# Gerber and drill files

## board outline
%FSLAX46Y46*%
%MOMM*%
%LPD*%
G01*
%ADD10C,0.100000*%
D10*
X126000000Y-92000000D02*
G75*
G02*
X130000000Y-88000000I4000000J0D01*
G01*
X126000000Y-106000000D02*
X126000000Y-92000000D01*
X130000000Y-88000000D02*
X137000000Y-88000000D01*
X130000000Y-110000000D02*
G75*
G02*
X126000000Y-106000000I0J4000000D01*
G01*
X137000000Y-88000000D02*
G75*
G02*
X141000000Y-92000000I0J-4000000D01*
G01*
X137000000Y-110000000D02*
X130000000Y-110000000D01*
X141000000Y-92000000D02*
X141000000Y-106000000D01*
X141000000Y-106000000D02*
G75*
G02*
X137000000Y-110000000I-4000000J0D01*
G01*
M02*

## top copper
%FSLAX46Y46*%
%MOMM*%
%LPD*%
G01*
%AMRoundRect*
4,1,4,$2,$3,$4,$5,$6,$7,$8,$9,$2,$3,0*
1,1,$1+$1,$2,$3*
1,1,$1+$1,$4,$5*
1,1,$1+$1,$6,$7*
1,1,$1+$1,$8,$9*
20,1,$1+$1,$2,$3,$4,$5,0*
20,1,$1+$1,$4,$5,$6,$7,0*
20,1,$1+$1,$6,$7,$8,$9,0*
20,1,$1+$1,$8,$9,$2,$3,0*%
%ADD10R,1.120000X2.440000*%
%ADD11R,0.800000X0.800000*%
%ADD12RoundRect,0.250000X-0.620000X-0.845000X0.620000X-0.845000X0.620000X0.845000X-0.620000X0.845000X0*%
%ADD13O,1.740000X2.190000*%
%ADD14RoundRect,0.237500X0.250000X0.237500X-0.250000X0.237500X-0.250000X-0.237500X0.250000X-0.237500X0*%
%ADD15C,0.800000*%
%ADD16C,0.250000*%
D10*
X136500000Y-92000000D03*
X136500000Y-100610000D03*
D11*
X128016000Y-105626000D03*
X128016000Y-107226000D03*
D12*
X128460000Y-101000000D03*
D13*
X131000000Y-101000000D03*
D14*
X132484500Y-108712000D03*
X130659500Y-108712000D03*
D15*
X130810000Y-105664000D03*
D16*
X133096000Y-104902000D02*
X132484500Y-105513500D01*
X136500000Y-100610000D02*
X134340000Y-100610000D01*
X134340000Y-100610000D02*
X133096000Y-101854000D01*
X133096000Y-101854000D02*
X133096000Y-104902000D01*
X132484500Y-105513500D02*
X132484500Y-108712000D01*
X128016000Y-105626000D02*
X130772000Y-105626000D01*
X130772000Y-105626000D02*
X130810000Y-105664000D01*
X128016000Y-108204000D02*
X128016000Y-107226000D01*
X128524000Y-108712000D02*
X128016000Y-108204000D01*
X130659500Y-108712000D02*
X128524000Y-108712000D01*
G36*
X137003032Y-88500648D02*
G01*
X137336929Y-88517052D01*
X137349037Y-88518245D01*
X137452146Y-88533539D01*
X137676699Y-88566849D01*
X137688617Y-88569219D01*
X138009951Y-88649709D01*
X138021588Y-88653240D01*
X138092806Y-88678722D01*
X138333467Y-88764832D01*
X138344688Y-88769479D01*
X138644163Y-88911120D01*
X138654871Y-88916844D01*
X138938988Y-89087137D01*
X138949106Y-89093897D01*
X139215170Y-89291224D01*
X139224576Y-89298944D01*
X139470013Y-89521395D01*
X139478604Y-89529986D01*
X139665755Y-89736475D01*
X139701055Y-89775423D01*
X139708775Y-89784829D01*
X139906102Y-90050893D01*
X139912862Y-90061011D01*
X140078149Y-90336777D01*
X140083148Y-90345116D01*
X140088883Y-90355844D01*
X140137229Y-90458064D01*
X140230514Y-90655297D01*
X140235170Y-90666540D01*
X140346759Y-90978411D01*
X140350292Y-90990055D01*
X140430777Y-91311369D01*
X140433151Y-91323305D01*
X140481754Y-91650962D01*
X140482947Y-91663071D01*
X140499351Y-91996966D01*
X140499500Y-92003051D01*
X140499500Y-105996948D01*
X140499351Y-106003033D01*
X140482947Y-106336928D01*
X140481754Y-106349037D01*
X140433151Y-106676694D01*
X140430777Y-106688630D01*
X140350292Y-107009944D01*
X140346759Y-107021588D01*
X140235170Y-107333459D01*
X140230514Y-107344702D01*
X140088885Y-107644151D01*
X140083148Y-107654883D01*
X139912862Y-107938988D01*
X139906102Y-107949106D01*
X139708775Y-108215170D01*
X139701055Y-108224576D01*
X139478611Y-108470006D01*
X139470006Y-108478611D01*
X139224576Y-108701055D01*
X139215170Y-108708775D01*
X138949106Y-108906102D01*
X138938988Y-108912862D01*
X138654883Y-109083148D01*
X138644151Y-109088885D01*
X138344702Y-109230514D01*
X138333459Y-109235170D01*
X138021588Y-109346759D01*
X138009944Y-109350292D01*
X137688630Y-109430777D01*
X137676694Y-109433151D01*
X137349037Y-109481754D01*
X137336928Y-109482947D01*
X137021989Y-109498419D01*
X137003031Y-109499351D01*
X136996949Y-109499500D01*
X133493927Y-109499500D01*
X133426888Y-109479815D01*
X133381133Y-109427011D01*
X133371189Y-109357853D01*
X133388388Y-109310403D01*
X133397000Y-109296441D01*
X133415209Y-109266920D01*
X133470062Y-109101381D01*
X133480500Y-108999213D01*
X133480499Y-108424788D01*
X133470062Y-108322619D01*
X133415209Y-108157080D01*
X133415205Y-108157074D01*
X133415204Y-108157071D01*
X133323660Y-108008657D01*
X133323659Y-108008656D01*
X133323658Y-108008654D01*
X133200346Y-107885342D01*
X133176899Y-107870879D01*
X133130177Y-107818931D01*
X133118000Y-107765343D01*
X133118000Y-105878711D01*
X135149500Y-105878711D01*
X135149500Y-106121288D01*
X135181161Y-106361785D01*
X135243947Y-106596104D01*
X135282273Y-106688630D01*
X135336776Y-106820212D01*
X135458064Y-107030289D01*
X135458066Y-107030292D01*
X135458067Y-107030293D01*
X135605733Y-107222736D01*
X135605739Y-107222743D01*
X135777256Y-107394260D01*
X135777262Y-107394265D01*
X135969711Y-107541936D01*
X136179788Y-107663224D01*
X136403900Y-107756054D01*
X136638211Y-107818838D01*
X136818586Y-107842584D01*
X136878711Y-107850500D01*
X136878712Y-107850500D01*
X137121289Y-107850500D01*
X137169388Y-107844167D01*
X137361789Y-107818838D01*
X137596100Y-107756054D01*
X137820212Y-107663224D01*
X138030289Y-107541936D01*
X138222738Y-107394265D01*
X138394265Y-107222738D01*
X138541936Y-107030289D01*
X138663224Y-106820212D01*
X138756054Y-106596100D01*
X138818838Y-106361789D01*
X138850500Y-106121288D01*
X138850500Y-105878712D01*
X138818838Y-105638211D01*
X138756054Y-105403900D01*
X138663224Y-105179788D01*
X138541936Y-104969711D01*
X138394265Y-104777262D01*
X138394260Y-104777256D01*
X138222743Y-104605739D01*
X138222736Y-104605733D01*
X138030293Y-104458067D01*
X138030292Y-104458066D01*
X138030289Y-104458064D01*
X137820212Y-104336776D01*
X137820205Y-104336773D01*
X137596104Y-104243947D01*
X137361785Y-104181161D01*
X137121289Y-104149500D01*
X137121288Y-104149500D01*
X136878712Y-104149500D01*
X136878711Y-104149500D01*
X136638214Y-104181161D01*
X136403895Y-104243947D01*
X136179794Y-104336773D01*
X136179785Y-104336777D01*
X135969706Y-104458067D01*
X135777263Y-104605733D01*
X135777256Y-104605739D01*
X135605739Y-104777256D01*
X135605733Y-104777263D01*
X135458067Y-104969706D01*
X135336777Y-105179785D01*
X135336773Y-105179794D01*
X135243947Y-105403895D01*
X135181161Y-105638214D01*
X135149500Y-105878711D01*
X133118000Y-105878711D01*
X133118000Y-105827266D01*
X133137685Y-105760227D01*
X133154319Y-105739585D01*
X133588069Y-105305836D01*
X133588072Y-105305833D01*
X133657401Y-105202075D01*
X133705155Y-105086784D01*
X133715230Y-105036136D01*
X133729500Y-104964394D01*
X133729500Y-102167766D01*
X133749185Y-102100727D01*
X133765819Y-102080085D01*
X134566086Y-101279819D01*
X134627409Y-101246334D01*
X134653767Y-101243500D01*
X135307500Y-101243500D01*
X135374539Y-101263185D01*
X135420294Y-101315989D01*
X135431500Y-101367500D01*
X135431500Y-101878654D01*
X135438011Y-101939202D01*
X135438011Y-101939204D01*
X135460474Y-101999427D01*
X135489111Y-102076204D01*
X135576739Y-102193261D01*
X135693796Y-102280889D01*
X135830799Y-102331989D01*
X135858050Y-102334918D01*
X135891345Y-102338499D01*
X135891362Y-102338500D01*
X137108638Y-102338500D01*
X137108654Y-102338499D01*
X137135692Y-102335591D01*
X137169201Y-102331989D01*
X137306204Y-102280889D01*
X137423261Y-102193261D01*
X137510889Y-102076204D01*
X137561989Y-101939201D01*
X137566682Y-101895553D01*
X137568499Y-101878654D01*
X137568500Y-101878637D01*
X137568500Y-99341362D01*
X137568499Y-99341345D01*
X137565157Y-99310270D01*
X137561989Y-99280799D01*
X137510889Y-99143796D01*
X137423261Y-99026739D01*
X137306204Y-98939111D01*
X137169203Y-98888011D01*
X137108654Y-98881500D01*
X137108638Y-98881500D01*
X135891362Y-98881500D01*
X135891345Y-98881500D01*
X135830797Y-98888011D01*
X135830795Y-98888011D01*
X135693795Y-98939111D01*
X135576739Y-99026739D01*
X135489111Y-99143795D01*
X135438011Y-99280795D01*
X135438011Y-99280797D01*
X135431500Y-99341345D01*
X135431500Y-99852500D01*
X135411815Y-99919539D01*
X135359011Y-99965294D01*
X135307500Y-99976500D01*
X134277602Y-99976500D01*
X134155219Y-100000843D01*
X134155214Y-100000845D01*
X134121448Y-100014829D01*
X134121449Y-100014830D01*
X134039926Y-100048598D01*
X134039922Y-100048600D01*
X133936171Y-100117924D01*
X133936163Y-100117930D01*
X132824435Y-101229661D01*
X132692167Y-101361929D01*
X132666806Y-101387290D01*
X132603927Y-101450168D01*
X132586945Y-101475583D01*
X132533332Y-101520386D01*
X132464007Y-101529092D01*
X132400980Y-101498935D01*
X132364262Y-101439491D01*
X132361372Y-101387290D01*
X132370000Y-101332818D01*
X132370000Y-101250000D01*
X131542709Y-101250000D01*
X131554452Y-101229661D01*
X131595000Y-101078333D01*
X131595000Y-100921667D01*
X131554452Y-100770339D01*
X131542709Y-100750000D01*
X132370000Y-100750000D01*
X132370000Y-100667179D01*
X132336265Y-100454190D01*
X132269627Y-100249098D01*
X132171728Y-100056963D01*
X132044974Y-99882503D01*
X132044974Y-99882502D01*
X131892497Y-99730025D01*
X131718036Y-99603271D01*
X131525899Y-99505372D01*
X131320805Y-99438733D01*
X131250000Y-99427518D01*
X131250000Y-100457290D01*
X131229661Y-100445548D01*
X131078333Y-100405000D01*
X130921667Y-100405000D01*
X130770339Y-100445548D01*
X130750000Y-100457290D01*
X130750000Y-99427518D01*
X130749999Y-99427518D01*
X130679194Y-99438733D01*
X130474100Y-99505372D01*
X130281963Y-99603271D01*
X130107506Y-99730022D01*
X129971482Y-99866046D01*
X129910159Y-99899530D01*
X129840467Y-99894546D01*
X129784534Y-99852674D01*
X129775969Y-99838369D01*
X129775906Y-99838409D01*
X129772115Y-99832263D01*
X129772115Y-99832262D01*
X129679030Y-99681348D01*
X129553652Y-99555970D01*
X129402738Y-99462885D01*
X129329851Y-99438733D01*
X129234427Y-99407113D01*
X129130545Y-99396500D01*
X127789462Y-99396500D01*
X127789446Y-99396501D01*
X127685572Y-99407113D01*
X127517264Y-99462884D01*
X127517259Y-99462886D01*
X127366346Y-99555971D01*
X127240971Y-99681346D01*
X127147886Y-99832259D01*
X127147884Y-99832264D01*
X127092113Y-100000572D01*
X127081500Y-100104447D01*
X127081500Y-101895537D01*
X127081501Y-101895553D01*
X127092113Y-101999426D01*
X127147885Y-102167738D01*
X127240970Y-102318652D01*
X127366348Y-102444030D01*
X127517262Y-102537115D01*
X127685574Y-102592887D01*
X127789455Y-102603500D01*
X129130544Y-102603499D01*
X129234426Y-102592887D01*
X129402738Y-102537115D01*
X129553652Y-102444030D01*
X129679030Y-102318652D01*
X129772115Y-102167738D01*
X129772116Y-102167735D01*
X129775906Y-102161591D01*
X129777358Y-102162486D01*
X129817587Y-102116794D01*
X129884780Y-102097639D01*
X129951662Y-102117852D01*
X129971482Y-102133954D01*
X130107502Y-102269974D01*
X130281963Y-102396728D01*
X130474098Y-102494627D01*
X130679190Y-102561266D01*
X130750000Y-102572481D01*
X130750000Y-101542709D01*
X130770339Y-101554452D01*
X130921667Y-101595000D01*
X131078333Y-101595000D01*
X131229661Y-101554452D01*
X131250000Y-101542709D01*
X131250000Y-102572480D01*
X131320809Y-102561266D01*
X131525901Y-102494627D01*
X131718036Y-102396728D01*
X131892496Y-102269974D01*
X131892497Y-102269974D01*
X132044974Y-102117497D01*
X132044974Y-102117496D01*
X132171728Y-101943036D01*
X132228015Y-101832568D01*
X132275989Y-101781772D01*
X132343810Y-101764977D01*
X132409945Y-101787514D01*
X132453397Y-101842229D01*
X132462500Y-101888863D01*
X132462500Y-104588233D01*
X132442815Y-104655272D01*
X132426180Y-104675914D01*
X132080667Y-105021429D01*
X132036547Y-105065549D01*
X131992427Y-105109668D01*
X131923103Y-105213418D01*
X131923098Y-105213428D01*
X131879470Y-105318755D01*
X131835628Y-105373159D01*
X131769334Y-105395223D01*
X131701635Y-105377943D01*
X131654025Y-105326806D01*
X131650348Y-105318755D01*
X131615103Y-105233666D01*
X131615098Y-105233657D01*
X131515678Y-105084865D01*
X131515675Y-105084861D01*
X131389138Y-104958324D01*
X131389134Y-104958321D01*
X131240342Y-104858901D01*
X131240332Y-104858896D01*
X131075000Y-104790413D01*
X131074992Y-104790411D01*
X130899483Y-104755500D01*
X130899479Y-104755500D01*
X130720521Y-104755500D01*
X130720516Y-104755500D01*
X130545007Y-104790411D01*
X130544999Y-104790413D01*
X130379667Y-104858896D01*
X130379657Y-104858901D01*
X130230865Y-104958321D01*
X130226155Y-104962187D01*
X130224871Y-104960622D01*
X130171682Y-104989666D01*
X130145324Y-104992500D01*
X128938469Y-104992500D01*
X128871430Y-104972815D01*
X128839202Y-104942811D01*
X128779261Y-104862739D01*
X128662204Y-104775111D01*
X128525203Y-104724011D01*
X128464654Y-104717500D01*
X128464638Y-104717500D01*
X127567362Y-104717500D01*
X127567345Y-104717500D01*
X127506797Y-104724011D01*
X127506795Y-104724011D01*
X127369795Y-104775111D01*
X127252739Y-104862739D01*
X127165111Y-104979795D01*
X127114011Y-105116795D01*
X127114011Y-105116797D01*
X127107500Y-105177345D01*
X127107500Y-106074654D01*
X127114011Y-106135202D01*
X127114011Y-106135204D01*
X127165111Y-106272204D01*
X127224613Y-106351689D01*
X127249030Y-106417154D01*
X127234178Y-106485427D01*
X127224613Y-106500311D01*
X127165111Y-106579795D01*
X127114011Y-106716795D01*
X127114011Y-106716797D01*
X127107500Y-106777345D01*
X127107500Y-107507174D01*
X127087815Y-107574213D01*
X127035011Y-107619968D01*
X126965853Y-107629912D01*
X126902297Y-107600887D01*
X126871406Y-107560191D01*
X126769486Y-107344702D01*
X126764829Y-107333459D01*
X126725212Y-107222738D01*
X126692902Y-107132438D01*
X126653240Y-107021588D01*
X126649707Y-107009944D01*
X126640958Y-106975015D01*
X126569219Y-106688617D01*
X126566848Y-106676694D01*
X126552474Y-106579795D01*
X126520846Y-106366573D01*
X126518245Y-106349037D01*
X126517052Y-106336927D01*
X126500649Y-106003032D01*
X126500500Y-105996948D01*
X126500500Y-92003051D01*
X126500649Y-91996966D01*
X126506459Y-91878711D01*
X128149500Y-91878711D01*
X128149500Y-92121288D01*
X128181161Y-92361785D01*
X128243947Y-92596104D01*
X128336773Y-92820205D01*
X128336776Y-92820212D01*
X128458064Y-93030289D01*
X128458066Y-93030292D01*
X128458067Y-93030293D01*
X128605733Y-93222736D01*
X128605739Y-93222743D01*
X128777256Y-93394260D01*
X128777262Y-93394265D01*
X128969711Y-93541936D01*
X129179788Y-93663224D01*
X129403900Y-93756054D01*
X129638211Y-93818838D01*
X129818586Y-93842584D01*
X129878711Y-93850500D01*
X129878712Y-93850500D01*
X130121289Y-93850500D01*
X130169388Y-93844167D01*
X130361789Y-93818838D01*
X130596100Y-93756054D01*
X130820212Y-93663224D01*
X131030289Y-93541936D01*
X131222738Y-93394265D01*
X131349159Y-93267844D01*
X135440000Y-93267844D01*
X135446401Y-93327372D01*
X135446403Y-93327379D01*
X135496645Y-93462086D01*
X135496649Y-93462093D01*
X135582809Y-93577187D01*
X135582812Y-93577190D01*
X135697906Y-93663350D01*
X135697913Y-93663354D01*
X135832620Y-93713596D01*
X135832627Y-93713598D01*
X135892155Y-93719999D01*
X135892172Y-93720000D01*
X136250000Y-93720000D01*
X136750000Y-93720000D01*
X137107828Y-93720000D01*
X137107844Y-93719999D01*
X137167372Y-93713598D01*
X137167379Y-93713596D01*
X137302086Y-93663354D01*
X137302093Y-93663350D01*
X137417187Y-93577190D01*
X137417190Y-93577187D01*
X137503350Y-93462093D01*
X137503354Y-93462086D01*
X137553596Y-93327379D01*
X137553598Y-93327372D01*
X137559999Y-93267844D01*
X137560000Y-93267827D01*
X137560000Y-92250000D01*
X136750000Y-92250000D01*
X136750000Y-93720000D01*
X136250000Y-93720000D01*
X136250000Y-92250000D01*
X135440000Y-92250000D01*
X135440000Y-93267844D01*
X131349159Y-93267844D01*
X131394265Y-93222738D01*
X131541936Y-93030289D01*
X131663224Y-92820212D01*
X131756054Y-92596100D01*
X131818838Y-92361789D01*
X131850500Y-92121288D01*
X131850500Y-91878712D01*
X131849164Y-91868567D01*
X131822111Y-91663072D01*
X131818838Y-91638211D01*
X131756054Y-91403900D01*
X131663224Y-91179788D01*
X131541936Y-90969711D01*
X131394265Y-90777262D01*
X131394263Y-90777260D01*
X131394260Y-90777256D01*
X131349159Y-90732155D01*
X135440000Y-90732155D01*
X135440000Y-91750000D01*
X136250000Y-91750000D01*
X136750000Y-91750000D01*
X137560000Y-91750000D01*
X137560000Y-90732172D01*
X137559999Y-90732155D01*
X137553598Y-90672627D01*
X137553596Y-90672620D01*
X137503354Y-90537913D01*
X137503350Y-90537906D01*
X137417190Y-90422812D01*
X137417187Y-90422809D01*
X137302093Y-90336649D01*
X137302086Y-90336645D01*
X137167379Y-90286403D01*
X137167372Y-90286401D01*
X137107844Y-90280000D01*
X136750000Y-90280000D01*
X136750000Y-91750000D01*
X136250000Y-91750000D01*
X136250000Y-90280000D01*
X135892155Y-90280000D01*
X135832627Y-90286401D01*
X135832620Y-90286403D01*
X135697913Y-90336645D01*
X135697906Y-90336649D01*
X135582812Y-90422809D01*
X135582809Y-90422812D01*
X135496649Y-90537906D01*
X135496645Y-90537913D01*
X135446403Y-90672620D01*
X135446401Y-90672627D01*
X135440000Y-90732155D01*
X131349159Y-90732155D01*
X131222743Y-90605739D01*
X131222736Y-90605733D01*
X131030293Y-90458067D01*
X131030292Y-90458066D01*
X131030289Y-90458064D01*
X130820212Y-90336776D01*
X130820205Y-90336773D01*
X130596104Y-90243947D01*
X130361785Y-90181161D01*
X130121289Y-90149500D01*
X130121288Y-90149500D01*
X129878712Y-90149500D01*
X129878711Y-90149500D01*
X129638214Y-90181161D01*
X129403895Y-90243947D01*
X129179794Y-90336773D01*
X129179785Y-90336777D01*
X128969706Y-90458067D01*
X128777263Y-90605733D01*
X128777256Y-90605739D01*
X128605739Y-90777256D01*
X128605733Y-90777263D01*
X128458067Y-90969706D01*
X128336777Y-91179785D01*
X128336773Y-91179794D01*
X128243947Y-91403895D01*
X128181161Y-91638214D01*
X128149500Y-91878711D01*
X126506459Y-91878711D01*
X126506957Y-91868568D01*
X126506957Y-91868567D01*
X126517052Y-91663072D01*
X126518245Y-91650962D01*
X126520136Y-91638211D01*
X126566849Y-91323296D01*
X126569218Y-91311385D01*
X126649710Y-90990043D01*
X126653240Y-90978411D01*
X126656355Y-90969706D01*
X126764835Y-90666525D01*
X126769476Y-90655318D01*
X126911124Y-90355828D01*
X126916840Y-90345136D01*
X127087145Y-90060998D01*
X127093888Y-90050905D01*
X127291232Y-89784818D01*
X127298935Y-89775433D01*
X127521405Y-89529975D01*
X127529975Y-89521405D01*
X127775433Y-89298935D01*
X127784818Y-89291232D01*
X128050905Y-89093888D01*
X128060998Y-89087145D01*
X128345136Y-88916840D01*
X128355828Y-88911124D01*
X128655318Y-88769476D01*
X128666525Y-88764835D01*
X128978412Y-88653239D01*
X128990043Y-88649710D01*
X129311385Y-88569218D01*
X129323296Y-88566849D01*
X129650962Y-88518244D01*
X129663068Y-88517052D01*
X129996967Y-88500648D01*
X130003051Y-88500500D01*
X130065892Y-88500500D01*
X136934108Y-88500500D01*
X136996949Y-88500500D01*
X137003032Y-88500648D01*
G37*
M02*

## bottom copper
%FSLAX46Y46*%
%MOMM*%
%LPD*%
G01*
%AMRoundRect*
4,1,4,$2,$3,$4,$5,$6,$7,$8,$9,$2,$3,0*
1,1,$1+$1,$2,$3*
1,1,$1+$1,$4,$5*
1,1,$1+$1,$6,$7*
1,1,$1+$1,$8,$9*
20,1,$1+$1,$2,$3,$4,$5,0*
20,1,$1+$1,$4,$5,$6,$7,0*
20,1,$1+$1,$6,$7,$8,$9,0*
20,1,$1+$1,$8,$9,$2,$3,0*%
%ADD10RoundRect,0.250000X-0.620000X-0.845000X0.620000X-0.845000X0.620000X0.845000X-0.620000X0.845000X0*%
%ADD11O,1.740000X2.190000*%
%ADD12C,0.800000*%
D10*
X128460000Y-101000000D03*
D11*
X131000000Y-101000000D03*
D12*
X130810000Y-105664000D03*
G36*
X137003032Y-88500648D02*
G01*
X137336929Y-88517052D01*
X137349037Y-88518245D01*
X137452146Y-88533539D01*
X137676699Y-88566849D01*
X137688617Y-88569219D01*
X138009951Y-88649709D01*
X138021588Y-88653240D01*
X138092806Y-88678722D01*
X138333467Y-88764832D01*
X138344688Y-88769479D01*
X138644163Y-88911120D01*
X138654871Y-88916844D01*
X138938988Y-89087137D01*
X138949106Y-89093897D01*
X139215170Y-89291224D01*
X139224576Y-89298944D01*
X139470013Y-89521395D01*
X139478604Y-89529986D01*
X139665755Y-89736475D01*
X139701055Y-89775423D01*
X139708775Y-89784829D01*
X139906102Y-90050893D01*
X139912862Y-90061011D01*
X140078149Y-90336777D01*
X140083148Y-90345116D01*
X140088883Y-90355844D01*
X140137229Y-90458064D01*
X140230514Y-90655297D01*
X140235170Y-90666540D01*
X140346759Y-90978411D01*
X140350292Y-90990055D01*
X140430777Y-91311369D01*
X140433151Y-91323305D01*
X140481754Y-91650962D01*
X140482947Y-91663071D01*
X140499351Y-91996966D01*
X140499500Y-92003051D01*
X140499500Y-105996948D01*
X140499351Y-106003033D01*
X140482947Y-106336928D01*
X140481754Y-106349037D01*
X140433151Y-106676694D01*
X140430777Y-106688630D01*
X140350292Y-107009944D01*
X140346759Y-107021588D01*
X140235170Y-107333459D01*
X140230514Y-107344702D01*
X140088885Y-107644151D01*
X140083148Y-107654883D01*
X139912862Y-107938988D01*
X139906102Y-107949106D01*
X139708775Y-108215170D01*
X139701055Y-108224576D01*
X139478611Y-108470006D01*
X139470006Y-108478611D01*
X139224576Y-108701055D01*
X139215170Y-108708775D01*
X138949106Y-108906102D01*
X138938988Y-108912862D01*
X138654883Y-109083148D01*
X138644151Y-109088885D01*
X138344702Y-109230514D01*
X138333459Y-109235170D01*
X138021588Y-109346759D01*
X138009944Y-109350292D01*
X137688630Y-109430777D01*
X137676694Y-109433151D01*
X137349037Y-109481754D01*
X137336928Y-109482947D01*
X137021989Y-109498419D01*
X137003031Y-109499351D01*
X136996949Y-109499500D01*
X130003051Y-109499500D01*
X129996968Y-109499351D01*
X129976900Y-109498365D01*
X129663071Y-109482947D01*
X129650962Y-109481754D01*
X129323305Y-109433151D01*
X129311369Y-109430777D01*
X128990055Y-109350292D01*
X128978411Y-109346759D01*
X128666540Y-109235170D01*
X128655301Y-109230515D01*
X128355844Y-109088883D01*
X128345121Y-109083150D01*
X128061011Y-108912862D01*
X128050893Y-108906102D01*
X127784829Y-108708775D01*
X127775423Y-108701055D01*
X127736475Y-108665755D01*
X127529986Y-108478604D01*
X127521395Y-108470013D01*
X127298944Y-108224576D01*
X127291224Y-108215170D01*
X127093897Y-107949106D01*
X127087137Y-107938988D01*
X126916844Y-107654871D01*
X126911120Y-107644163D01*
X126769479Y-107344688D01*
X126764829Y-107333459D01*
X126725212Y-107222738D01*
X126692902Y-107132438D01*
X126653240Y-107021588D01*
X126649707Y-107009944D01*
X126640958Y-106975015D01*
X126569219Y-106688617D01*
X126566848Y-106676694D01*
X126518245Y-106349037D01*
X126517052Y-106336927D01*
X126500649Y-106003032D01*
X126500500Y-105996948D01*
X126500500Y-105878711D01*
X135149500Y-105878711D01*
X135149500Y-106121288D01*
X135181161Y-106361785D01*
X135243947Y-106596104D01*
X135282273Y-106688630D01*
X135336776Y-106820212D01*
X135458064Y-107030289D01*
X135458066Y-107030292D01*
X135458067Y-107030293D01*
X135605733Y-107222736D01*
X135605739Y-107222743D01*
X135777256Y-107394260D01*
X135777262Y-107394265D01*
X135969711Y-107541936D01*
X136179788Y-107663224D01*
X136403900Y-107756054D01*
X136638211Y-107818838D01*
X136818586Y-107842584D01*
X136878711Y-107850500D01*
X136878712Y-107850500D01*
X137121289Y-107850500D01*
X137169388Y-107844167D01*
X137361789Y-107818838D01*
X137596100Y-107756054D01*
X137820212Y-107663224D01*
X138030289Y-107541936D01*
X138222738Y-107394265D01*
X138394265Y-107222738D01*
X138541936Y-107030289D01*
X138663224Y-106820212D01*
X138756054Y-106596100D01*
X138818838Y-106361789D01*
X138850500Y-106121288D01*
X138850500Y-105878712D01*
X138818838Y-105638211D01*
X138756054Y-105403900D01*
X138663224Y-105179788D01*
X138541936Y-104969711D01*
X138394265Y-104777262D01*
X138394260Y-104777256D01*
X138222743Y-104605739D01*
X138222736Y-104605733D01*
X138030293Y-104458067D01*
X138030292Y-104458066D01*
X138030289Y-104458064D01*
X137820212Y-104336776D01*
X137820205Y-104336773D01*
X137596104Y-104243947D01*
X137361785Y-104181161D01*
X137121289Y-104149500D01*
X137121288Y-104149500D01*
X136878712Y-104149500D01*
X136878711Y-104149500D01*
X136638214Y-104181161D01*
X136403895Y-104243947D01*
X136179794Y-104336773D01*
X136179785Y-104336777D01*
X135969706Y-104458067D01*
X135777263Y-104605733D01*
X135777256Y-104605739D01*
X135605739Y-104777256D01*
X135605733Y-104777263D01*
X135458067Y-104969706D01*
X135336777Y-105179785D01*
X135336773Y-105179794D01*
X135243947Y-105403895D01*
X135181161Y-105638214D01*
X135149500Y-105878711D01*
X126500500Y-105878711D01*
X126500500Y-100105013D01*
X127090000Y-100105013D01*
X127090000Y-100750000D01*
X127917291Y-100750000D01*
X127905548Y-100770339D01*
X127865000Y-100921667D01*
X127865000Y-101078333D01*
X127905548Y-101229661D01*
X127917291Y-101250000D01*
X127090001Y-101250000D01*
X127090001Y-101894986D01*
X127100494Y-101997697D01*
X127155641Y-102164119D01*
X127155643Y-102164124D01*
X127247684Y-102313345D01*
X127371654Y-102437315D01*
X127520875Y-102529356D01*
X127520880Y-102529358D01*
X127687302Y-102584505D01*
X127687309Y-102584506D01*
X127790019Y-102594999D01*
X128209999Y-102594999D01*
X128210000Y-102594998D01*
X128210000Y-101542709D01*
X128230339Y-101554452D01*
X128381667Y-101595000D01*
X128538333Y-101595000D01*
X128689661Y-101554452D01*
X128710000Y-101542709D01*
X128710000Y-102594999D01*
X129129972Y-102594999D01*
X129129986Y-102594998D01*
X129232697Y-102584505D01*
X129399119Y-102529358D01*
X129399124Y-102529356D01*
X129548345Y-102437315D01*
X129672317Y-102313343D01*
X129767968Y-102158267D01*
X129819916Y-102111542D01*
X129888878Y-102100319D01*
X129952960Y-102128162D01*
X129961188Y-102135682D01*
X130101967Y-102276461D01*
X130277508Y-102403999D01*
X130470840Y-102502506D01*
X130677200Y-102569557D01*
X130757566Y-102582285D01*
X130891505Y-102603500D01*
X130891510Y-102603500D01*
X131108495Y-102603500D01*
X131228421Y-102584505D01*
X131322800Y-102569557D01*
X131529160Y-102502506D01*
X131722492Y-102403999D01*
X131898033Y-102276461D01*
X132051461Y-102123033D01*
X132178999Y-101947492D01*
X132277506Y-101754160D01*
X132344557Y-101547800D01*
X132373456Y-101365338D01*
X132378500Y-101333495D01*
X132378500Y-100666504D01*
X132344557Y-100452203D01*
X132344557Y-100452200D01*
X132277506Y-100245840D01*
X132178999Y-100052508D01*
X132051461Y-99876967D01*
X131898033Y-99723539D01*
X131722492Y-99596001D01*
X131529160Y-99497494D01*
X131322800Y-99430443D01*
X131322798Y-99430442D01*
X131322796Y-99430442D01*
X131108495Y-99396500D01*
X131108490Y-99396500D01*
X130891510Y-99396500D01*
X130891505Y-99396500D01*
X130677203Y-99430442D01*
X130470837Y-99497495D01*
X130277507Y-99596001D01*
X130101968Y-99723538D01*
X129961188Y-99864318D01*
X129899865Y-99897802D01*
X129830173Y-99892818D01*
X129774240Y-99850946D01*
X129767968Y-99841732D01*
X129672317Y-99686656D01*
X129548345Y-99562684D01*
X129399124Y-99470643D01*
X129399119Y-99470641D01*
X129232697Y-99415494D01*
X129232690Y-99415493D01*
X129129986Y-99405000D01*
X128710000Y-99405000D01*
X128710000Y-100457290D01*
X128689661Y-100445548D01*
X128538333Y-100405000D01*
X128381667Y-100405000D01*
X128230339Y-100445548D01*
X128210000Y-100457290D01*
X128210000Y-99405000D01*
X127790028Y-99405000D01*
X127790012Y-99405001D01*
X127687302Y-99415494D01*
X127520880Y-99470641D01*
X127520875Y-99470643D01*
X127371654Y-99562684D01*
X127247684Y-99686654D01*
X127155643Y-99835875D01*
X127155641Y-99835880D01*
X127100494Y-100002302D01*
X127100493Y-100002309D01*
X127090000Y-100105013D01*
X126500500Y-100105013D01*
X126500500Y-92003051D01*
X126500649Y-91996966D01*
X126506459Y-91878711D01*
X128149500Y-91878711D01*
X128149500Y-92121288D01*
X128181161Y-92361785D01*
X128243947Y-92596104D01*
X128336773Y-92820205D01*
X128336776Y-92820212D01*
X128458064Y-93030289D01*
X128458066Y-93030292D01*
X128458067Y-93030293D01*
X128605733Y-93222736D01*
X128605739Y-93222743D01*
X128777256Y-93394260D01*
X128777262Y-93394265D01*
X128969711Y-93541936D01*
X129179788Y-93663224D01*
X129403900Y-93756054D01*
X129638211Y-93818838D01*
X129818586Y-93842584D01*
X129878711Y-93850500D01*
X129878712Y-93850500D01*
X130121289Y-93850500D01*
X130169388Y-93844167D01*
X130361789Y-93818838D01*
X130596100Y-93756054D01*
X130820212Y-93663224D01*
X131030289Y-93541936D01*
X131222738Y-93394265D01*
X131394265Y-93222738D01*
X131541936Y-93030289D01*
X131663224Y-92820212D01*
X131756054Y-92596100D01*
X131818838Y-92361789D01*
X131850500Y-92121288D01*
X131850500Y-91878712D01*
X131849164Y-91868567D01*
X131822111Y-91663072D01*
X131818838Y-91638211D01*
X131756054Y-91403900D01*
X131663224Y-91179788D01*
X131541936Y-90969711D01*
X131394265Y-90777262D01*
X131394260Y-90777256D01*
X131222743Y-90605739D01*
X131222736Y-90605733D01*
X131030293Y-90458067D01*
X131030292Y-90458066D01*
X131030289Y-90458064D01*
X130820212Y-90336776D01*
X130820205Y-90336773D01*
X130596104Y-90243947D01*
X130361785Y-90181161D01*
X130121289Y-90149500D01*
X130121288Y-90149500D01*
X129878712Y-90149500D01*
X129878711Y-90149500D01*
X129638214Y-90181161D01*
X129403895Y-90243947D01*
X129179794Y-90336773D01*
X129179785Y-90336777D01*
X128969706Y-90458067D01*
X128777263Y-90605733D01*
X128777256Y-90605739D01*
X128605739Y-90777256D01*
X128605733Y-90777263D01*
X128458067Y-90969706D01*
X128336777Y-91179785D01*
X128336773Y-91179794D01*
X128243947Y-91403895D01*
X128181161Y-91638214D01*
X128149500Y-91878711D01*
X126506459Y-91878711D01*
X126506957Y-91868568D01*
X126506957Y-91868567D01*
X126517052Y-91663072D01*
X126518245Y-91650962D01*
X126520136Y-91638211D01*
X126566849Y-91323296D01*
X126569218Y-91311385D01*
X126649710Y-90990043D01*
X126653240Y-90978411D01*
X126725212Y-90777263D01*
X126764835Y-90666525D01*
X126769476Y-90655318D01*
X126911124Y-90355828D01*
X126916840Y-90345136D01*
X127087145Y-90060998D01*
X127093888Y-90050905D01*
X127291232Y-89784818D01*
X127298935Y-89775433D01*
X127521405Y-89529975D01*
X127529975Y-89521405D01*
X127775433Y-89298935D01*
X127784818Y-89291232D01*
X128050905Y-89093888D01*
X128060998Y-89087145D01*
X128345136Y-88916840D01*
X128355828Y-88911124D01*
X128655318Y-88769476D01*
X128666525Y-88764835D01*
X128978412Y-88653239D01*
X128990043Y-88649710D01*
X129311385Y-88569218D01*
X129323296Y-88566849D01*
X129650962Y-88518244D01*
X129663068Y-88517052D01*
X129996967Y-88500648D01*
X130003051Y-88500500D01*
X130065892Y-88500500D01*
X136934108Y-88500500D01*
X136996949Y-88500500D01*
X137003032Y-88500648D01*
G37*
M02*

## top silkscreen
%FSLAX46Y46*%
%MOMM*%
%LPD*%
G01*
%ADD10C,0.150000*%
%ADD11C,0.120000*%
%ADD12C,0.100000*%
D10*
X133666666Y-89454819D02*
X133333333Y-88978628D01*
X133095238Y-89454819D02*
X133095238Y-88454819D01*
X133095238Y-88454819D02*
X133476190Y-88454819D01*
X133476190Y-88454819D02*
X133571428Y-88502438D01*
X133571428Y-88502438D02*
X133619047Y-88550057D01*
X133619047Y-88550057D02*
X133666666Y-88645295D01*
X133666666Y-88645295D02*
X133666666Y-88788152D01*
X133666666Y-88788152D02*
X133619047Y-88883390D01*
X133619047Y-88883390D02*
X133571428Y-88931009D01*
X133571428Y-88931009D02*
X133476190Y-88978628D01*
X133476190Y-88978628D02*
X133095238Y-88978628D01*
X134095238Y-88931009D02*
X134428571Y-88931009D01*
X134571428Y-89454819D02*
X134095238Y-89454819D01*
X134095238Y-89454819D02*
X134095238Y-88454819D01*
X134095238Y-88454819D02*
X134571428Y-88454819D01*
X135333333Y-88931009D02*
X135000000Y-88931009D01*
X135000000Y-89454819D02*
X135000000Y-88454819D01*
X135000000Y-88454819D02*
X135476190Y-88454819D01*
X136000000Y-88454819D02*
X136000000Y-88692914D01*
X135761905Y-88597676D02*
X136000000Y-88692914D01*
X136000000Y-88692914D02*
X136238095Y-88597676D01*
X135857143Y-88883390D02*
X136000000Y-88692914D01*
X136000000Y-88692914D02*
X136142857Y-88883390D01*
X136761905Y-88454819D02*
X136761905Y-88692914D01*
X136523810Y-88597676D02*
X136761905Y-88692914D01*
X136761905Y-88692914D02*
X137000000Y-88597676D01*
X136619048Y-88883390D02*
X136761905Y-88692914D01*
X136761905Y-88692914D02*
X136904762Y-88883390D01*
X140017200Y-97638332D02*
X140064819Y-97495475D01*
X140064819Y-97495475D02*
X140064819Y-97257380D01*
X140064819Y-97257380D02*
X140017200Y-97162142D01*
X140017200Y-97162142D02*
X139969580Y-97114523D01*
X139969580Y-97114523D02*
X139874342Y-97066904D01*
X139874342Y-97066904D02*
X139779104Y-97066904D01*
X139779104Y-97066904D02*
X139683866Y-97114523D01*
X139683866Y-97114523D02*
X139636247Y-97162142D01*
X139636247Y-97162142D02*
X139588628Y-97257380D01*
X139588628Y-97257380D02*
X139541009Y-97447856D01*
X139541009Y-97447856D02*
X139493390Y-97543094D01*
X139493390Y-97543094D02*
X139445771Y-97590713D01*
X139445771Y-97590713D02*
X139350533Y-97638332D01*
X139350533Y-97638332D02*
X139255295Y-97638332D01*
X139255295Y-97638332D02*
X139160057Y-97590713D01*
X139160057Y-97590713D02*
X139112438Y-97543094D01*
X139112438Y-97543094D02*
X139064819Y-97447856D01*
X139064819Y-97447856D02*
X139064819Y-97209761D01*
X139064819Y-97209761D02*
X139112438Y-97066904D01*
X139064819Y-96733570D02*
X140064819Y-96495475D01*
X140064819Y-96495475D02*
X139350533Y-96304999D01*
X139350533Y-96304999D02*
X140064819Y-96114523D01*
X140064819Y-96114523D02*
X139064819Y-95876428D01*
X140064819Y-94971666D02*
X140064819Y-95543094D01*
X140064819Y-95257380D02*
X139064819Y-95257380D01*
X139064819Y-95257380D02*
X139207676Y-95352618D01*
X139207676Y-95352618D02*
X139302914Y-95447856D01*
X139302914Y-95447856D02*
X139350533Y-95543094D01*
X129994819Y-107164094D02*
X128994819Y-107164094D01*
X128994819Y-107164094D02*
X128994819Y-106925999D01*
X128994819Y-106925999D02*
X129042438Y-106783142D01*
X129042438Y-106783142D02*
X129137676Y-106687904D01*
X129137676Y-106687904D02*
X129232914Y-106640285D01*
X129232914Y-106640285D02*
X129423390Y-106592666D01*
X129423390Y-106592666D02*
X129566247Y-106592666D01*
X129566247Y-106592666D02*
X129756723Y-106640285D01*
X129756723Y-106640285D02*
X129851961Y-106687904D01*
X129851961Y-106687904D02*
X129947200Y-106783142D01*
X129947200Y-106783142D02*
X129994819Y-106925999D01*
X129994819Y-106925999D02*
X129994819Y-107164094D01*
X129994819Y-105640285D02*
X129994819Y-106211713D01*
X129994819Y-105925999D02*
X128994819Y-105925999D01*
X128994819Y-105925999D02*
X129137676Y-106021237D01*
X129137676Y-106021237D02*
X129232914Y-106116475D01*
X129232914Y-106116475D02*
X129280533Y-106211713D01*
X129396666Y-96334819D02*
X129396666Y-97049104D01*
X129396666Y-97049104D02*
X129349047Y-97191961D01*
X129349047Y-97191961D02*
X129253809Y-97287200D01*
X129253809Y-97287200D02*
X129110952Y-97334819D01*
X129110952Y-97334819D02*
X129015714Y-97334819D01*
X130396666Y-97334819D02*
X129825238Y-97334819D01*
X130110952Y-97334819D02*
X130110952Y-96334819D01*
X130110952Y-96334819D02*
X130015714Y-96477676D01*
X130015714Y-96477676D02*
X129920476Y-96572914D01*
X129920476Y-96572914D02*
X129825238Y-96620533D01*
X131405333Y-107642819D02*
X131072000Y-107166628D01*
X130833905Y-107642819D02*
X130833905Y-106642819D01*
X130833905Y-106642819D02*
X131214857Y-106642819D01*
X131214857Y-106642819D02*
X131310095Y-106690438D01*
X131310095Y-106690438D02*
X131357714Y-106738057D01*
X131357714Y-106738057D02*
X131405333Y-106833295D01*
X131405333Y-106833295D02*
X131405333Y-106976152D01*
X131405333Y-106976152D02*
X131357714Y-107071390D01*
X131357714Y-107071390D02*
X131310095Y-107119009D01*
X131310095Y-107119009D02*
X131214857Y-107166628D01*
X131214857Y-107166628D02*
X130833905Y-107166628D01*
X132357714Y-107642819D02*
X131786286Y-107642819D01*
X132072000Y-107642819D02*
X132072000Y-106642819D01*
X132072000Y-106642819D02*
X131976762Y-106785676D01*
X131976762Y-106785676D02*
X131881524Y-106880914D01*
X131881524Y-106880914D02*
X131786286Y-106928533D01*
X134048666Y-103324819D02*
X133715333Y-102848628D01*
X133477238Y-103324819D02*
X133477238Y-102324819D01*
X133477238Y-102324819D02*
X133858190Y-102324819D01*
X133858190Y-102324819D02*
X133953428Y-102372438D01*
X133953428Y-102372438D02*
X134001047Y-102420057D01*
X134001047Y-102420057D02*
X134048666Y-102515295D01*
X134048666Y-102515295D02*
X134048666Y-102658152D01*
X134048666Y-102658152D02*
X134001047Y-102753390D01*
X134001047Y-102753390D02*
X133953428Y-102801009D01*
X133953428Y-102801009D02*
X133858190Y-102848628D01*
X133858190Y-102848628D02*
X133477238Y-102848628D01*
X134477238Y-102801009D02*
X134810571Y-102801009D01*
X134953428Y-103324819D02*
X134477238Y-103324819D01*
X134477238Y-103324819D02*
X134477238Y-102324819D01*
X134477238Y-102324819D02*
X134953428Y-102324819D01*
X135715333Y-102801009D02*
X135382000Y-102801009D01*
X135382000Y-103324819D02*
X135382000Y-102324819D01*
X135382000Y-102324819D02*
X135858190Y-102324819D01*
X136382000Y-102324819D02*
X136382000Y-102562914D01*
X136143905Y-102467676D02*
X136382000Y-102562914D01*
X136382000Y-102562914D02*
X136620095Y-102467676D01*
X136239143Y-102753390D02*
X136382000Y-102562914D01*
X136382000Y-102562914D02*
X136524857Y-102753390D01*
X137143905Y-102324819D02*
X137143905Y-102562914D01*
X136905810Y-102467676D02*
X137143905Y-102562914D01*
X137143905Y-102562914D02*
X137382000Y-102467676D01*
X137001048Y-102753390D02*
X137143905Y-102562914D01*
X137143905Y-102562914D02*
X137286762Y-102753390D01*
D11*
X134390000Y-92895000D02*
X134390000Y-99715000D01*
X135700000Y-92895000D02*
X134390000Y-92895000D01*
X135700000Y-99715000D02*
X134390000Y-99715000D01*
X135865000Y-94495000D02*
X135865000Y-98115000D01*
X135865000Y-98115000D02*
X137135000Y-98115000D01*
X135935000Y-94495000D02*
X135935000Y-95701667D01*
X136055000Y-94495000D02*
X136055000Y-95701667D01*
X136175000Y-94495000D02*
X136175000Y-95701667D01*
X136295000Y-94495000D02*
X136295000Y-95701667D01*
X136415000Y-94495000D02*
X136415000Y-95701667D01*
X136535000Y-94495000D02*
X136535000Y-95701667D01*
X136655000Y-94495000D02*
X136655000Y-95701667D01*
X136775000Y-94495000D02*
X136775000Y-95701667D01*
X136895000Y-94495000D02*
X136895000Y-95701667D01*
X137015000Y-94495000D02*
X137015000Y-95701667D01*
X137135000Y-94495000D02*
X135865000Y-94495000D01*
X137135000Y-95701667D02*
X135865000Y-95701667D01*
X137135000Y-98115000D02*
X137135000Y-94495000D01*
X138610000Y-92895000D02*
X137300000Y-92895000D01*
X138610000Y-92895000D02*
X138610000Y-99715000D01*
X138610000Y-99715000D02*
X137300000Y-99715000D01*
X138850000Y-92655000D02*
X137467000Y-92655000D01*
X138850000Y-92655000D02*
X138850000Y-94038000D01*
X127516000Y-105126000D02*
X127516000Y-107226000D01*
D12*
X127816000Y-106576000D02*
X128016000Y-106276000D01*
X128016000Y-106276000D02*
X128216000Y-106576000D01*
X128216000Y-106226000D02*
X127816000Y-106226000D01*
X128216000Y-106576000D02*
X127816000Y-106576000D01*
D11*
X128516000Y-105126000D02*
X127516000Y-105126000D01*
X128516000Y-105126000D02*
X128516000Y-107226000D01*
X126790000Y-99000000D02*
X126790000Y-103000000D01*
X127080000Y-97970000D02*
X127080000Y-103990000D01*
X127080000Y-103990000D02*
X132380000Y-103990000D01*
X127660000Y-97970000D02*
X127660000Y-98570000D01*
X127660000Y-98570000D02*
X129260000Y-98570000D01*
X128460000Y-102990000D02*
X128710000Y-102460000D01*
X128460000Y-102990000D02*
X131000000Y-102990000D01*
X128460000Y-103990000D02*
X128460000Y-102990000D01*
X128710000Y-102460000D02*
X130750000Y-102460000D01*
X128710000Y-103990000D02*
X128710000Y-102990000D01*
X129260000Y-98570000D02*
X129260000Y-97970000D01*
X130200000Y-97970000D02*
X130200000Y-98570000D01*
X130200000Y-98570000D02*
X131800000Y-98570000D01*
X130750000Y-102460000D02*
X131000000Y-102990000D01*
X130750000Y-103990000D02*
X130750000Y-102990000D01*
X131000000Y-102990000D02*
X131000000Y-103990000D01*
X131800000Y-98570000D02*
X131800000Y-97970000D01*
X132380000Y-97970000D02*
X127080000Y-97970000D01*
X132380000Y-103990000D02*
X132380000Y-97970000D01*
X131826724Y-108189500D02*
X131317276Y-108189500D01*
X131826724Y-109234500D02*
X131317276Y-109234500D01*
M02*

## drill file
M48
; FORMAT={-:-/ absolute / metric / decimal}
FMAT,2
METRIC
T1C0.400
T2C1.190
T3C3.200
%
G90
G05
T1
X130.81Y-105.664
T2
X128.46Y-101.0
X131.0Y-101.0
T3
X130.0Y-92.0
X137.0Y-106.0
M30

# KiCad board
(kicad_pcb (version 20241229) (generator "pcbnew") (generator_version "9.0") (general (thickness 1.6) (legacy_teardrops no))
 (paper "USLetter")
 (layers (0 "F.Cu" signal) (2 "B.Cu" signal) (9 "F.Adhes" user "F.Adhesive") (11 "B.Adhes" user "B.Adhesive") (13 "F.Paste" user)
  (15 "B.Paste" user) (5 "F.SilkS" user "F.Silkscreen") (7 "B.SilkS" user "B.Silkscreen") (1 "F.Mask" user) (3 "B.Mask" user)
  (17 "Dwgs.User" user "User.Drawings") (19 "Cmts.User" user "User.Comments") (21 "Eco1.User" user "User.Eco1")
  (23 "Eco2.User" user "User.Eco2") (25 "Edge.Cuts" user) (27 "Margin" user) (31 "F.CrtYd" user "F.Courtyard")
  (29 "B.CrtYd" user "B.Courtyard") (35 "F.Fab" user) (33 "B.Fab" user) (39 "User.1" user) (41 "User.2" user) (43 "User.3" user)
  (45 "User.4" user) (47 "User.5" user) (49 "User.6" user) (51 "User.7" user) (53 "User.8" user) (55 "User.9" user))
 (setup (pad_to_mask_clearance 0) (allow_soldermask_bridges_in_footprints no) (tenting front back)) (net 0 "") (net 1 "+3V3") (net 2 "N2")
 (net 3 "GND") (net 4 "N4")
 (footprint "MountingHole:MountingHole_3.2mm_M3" (layer "F.Cu") (at 130 92)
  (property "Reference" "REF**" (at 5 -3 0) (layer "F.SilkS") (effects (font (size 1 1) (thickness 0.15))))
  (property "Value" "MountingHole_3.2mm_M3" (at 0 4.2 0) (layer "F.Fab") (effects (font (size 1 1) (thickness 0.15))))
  (pad "" np_thru_hole circle (at 0 0) (size 3.2 3.2) (drill 3.2) (layers "*.Cu" "*.Mask")))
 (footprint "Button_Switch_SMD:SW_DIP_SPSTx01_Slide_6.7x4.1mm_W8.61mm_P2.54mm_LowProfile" (layer "F.Cu") (at 136.5 96.305 -90)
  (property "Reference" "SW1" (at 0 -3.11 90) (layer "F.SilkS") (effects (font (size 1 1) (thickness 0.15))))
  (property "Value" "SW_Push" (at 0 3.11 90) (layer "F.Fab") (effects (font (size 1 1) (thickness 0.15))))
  (fp_line (start -3.41 2.11) (end 3.41 2.11) (stroke (width 0.12) (type solid)) (layer "F.SilkS"))
  (fp_line (start -3.41 0.8) (end -3.41 2.11) (stroke (width 0.12) (type solid)) (layer "F.SilkS"))
  (fp_line (start 3.41 0.8) (end 3.41 2.11) (stroke (width 0.12) (type solid)) (layer "F.SilkS"))
  (fp_line (start -1.81 0.635) (end 1.81 0.635) (stroke (width 0.12) (type solid)) (layer "F.SilkS"))
  (fp_line (start 1.81 0.635) (end 1.81 -0.635) (stroke (width 0.12) (type solid)) (layer "F.SilkS"))
  (fp_line (start -1.81 0.565) (end -0.603333 0.565) (stroke (width 0.12) (type solid)) (layer "F.SilkS"))
  (fp_line (start -1.81 0.445) (end -0.603333 0.445) (stroke (width 0.12) (type solid)) (layer "F.SilkS"))
  (fp_line (start -1.81 0.325) (end -0.603333 0.325) (stroke (width 0.12) (type solid)) (layer "F.SilkS"))
  (fp_line (start -1.81 0.205) (end -0.603333 0.205) (stroke (width 0.12) (type solid)) (layer "F.SilkS"))
  (fp_line (start -1.81 0.085) (end -0.603333 0.085) (stroke (width 0.12) (type solid)) (layer "F.SilkS"))
  (fp_line (start -1.81 -0.035) (end -0.603333 -0.035) (stroke (width 0.12) (type solid)) (layer "F.SilkS"))
  (fp_line (start -1.81 -0.155) (end -0.603333 -0.155) (stroke (width 0.12) (type solid)) (layer "F.SilkS"))
  (fp_line (start -1.81 -0.275) (end -0.603333 -0.275) (stroke (width 0.12) (type solid)) (layer "F.SilkS"))
  (fp_line (start -1.81 -0.395) (end -0.603333 -0.395) (stroke (width 0.12) (type solid)) (layer "F.SilkS"))
  (fp_line (start -1.81 -0.515) (end -0.603333 -0.515) (stroke (width 0.12) (type solid)) (layer "F.SilkS"))
  (fp_line (start -1.81 -0.635) (end -1.81 0.635) (stroke (width 0.12) (type solid)) (layer "F.SilkS"))
  (fp_line (start -0.603333 -0.635) (end -0.603333 0.635) (stroke (width 0.12) (type solid)) (layer "F.SilkS"))
  (fp_line (start 1.81 -0.635) (end -1.81 -0.635) (stroke (width 0.12) (type solid)) (layer "F.SilkS"))
  (fp_line (start -3.41 -2.11) (end -3.41 -0.8) (stroke (width 0.12) (type solid)) (layer "F.SilkS"))
  (fp_line (start -3.41 -2.11) (end 3.41 -2.11) (stroke (width 0.12) (type solid)) (layer "F.SilkS"))
  (fp_line (start 3.41 -2.11) (end 3.41 -0.8) (stroke (width 0.12) (type solid)) (layer "F.SilkS"))
  (fp_line (start -3.65 -2.35) (end -3.65 -0.967) (stroke (width 0.12) (type solid)) (layer "F.SilkS"))
  (fp_line (start -3.65 -2.35) (end -2.267 -2.35) (stroke (width 0.12) (type solid)) (layer "F.SilkS"))
  (pad "1" smd rect (at -4.305 0 270) (size 2.44 1.12) (layers "F.Cu" "F.Mask" "F.Paste") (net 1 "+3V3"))
  (pad "2" smd rect (at 4.305 0 270) (size 2.44 1.12) (layers "F.Cu" "F.Mask" "F.Paste") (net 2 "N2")))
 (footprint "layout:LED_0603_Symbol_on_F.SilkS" (layer "F.Cu") (at 128.016 106.426 -90)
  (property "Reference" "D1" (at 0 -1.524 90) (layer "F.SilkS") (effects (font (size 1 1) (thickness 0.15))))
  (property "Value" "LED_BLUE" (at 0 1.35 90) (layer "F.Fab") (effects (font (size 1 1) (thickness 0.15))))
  (fp_line (start -1.3 0.5) (end 0.8 0.5) (stroke (width 0.12) (type solid)) (layer "F.SilkS"))
  (fp_line (start 0.15 0.2) (end -0.15 0) (stroke (width 0.1) (type solid)) (layer "F.SilkS"))
  (fp_line (start -0.15 0) (end 0.15 -0.2) (stroke (width 0.1) (type solid)) (layer "F.SilkS"))
  (fp_line (start -0.2 -0.2) (end -0.2 0.2) (stroke (width 0.1) (type solid)) (layer "F.SilkS"))
  (fp_line (start 0.15 -0.2) (end 0.15 0.2) (stroke (width 0.1) (type solid)) (layer "F.SilkS"))
  (fp_line (start -1.3 -0.5) (end -1.3 0.5) (stroke (width 0.12) (type solid)) (layer "F.SilkS"))
  (fp_line (start -1.3 -0.5) (end 0.8 -0.5) (stroke (width 0.12) (type solid)) (layer "F.SilkS"))
  (pad "1" smd rect (at -0.8 0 90) (size 0.8 0.8) (layers "F.Cu" "F.Mask" "F.Paste") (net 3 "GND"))
  (pad "2" smd rect (at 0.8 0 90) (size 0.8 0.8) (layers "F.Cu" "F.Mask" "F.Paste") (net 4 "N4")))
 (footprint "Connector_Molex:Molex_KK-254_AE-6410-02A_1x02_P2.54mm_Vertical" (layer "F.Cu") (at 128.46 101)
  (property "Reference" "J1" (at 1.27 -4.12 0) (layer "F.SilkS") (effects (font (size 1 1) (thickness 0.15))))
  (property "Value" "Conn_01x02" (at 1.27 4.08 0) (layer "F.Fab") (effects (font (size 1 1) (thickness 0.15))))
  (fp_line (start -1.67 -2) (end -1.67 2) (stroke (width 0.12) (type solid)) (layer "F.SilkS"))
  (fp_line (start -1.38 -3.03) (end -1.38 2.99) (stroke (width 0.12) (type solid)) (layer "F.SilkS"))
  (fp_line (start -1.38 2.99) (end 3.92 2.99) (stroke (width 0.12) (type solid)) (layer "F.SilkS"))
  (fp_line (start -0.8 -3.03) (end -0.8 -2.43) (stroke (width 0.12) (type solid)) (layer "F.SilkS"))
  (fp_line (start -0.8 -2.43) (end 0.8 -2.43) (stroke (width 0.12) (type solid)) (layer "F.SilkS"))
  (fp_line (start 0 1.99) (end 0.25 1.46) (stroke (width 0.12) (type solid)) (layer "F.SilkS"))
  (fp_line (start 0 1.99) (end 2.54 1.99) (stroke (width 0.12) (type solid)) (layer "F.SilkS"))
  (fp_line (start 0 2.99) (end 0 1.99) (stroke (width 0.12) (type solid)) (layer "F.SilkS"))
  (fp_line (start 0.25 1.46) (end 2.29 1.46) (stroke (width 0.12) (type solid)) (layer "F.SilkS"))
  (fp_line (start 0.25 2.99) (end 0.25 1.99) (stroke (width 0.12) (type solid)) (layer "F.SilkS"))
  (fp_line (start 0.8 -2.43) (end 0.8 -3.03) (stroke (width 0.12) (type solid)) (layer "F.SilkS"))
  (fp_line (start 1.74 -3.03) (end 1.74 -2.43) (stroke (width 0.12) (type solid)) (layer "F.SilkS"))
  (fp_line (start 1.74 -2.43) (end 3.34 -2.43) (stroke (width 0.12) (type solid)) (layer "F.SilkS"))
  (fp_line (start 2.29 1.46) (end 2.54 1.99) (stroke (width 0.12) (type solid)) (layer "F.SilkS"))
  (fp_line (start 2.29 2.99) (end 2.29 1.99) (stroke (width 0.12) (type solid)) (layer "F.SilkS"))
  (fp_line (start 2.54 1.99) (end 2.54 2.99) (stroke (width 0.12) (type solid)) (layer "F.SilkS"))
  (fp_line (start 3.34 -2.43) (end 3.34 -3.03) (stroke (width 0.12) (type solid)) (layer "F.SilkS"))
  (fp_line (start 3.92 -3.03) (end -1.38 -3.03) (stroke (width 0.12) (type solid)) (layer "F.SilkS"))
  (fp_line (start 3.92 2.99) (end 3.92 -3.03) (stroke (width 0.12) (type solid)) (layer "F.SilkS"))
  (pad "1" thru_hole roundrect (at 0 0) (size 1.74 2.19) (drill 1.19) (layers "*.Cu" "*.Mask") (remove_unused_layers no)
   (roundrect_rratio 0.143678) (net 3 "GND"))
  (pad "2" thru_hole oval (at 2.54 0) (size 1.74 2.19) (drill 1.19) (layers "*.Cu" "*.Mask") (remove_unused_layers no) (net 1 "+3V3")))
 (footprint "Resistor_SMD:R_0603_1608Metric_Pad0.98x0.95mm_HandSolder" (layer "F.Cu") (at 131.572 108.712 180)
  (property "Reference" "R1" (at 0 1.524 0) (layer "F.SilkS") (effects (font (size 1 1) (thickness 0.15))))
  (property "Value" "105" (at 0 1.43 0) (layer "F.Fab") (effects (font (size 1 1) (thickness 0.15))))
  (fp_line (start -0.254724 0.5225) (end 0.254724 0.5225) (stroke (width 0.12) (type solid)) (layer "F.SilkS"))
  (fp_line (start -0.254724 -0.5225) (end 0.254724 -0.5225) (stroke (width 0.12) (type solid)) (layer "F.SilkS"))
  (pad "1" smd roundrect (at -0.9125 0 180) (size 0.975 0.95) (layers "F.Cu" "F.Mask" "F.Paste") (roundrect_rratio 0.25) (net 2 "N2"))
  (pad "2" smd roundrect (at 0.9125 0 180) (size 0.975 0.95) (layers "F.Cu" "F.Mask" "F.Paste") (roundrect_rratio 0.25) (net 4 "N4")))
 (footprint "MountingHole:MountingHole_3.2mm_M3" (layer "F.Cu") (at 137 106)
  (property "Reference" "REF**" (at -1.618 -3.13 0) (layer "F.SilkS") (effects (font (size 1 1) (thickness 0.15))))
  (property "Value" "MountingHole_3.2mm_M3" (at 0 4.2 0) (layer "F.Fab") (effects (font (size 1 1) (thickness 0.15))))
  (pad "" np_thru_hole circle (at 0 0) (size 3.2 3.2) (drill 3.2) (layers "*.Cu" "*.Mask")))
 (gr_arc (start 126 92) (mid 127.171573 89.171573) (end 130 88) (stroke (width 0.1) (type default)) (layer "Edge.Cuts"))
 (gr_line (start 126 106) (end 126 92) (stroke (width 0.1) (type default)) (layer "Edge.Cuts"))
 (gr_line (start 130 88) (end 137 88) (stroke (width 0.1) (type default)) (layer "Edge.Cuts"))
 (gr_arc (start 130 110) (mid 127.171573 108.828427) (end 126 106) (stroke (width 0.1) (type default)) (layer "Edge.Cuts"))
 (gr_arc (start 137 88) (mid 139.828427 89.171573) (end 141 92) (stroke (width 0.1) (type default)) (layer "Edge.Cuts"))
 (gr_line (start 137 110) (end 130 110) (stroke (width 0.1) (type default)) (layer "Edge.Cuts"))
 (gr_line (start 141 92) (end 141 106) (stroke (width 0.1) (type default)) (layer "Edge.Cuts"))
 (gr_arc (start 141 106) (mid 139.828427 108.828427) (end 137 110) (stroke (width 0.1) (type default)) (layer "Edge.Cuts"))
 (segment (start 133.096 104.902) (end 132.4845 105.5135) (width 0.25) (layer "F.Cu") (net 2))
 (segment (start 136.5 100.61) (end 134.34 100.61) (width 0.25) (layer "F.Cu") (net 2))
 (segment (start 134.34 100.61) (end 133.096 101.854) (width 0.25) (layer "F.Cu") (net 2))
 (segment (start 133.096 101.854) (end 133.096 104.902) (width 0.25) (layer "F.Cu") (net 2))
 (segment (start 132.4845 105.5135) (end 132.4845 108.712) (width 0.25) (layer "F.Cu") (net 2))
 (segment (start 128.016 105.626) (end 130.772 105.626) (width 0.25) (layer "F.Cu") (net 3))
 (segment (start 130.772 105.626) (end 130.81 105.664) (width 0.25) (layer "F.Cu") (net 3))
 (via (at 130.81 105.664) (size 0.8) (drill 0.4) (layers "F.Cu" "B.Cu") (free yes) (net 3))
 (segment (start 128.016 108.204) (end 128.016 107.226) (width 0.25) (layer "F.Cu") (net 4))
 (segment (start 128.524 108.712) (end 128.016 108.204) (width 0.25) (layer "F.Cu") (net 4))
 (segment (start 130.6595 108.712) (end 128.524 108.712) (width 0.25) (layer "F.Cu") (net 4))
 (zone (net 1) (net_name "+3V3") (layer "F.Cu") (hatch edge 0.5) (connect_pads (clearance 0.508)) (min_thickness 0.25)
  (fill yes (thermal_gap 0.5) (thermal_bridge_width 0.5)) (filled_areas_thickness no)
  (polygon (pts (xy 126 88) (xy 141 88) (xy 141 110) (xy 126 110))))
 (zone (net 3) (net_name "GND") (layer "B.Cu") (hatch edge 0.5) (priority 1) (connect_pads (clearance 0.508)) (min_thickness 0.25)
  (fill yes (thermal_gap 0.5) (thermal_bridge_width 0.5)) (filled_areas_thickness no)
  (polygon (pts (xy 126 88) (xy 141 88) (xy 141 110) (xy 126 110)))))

